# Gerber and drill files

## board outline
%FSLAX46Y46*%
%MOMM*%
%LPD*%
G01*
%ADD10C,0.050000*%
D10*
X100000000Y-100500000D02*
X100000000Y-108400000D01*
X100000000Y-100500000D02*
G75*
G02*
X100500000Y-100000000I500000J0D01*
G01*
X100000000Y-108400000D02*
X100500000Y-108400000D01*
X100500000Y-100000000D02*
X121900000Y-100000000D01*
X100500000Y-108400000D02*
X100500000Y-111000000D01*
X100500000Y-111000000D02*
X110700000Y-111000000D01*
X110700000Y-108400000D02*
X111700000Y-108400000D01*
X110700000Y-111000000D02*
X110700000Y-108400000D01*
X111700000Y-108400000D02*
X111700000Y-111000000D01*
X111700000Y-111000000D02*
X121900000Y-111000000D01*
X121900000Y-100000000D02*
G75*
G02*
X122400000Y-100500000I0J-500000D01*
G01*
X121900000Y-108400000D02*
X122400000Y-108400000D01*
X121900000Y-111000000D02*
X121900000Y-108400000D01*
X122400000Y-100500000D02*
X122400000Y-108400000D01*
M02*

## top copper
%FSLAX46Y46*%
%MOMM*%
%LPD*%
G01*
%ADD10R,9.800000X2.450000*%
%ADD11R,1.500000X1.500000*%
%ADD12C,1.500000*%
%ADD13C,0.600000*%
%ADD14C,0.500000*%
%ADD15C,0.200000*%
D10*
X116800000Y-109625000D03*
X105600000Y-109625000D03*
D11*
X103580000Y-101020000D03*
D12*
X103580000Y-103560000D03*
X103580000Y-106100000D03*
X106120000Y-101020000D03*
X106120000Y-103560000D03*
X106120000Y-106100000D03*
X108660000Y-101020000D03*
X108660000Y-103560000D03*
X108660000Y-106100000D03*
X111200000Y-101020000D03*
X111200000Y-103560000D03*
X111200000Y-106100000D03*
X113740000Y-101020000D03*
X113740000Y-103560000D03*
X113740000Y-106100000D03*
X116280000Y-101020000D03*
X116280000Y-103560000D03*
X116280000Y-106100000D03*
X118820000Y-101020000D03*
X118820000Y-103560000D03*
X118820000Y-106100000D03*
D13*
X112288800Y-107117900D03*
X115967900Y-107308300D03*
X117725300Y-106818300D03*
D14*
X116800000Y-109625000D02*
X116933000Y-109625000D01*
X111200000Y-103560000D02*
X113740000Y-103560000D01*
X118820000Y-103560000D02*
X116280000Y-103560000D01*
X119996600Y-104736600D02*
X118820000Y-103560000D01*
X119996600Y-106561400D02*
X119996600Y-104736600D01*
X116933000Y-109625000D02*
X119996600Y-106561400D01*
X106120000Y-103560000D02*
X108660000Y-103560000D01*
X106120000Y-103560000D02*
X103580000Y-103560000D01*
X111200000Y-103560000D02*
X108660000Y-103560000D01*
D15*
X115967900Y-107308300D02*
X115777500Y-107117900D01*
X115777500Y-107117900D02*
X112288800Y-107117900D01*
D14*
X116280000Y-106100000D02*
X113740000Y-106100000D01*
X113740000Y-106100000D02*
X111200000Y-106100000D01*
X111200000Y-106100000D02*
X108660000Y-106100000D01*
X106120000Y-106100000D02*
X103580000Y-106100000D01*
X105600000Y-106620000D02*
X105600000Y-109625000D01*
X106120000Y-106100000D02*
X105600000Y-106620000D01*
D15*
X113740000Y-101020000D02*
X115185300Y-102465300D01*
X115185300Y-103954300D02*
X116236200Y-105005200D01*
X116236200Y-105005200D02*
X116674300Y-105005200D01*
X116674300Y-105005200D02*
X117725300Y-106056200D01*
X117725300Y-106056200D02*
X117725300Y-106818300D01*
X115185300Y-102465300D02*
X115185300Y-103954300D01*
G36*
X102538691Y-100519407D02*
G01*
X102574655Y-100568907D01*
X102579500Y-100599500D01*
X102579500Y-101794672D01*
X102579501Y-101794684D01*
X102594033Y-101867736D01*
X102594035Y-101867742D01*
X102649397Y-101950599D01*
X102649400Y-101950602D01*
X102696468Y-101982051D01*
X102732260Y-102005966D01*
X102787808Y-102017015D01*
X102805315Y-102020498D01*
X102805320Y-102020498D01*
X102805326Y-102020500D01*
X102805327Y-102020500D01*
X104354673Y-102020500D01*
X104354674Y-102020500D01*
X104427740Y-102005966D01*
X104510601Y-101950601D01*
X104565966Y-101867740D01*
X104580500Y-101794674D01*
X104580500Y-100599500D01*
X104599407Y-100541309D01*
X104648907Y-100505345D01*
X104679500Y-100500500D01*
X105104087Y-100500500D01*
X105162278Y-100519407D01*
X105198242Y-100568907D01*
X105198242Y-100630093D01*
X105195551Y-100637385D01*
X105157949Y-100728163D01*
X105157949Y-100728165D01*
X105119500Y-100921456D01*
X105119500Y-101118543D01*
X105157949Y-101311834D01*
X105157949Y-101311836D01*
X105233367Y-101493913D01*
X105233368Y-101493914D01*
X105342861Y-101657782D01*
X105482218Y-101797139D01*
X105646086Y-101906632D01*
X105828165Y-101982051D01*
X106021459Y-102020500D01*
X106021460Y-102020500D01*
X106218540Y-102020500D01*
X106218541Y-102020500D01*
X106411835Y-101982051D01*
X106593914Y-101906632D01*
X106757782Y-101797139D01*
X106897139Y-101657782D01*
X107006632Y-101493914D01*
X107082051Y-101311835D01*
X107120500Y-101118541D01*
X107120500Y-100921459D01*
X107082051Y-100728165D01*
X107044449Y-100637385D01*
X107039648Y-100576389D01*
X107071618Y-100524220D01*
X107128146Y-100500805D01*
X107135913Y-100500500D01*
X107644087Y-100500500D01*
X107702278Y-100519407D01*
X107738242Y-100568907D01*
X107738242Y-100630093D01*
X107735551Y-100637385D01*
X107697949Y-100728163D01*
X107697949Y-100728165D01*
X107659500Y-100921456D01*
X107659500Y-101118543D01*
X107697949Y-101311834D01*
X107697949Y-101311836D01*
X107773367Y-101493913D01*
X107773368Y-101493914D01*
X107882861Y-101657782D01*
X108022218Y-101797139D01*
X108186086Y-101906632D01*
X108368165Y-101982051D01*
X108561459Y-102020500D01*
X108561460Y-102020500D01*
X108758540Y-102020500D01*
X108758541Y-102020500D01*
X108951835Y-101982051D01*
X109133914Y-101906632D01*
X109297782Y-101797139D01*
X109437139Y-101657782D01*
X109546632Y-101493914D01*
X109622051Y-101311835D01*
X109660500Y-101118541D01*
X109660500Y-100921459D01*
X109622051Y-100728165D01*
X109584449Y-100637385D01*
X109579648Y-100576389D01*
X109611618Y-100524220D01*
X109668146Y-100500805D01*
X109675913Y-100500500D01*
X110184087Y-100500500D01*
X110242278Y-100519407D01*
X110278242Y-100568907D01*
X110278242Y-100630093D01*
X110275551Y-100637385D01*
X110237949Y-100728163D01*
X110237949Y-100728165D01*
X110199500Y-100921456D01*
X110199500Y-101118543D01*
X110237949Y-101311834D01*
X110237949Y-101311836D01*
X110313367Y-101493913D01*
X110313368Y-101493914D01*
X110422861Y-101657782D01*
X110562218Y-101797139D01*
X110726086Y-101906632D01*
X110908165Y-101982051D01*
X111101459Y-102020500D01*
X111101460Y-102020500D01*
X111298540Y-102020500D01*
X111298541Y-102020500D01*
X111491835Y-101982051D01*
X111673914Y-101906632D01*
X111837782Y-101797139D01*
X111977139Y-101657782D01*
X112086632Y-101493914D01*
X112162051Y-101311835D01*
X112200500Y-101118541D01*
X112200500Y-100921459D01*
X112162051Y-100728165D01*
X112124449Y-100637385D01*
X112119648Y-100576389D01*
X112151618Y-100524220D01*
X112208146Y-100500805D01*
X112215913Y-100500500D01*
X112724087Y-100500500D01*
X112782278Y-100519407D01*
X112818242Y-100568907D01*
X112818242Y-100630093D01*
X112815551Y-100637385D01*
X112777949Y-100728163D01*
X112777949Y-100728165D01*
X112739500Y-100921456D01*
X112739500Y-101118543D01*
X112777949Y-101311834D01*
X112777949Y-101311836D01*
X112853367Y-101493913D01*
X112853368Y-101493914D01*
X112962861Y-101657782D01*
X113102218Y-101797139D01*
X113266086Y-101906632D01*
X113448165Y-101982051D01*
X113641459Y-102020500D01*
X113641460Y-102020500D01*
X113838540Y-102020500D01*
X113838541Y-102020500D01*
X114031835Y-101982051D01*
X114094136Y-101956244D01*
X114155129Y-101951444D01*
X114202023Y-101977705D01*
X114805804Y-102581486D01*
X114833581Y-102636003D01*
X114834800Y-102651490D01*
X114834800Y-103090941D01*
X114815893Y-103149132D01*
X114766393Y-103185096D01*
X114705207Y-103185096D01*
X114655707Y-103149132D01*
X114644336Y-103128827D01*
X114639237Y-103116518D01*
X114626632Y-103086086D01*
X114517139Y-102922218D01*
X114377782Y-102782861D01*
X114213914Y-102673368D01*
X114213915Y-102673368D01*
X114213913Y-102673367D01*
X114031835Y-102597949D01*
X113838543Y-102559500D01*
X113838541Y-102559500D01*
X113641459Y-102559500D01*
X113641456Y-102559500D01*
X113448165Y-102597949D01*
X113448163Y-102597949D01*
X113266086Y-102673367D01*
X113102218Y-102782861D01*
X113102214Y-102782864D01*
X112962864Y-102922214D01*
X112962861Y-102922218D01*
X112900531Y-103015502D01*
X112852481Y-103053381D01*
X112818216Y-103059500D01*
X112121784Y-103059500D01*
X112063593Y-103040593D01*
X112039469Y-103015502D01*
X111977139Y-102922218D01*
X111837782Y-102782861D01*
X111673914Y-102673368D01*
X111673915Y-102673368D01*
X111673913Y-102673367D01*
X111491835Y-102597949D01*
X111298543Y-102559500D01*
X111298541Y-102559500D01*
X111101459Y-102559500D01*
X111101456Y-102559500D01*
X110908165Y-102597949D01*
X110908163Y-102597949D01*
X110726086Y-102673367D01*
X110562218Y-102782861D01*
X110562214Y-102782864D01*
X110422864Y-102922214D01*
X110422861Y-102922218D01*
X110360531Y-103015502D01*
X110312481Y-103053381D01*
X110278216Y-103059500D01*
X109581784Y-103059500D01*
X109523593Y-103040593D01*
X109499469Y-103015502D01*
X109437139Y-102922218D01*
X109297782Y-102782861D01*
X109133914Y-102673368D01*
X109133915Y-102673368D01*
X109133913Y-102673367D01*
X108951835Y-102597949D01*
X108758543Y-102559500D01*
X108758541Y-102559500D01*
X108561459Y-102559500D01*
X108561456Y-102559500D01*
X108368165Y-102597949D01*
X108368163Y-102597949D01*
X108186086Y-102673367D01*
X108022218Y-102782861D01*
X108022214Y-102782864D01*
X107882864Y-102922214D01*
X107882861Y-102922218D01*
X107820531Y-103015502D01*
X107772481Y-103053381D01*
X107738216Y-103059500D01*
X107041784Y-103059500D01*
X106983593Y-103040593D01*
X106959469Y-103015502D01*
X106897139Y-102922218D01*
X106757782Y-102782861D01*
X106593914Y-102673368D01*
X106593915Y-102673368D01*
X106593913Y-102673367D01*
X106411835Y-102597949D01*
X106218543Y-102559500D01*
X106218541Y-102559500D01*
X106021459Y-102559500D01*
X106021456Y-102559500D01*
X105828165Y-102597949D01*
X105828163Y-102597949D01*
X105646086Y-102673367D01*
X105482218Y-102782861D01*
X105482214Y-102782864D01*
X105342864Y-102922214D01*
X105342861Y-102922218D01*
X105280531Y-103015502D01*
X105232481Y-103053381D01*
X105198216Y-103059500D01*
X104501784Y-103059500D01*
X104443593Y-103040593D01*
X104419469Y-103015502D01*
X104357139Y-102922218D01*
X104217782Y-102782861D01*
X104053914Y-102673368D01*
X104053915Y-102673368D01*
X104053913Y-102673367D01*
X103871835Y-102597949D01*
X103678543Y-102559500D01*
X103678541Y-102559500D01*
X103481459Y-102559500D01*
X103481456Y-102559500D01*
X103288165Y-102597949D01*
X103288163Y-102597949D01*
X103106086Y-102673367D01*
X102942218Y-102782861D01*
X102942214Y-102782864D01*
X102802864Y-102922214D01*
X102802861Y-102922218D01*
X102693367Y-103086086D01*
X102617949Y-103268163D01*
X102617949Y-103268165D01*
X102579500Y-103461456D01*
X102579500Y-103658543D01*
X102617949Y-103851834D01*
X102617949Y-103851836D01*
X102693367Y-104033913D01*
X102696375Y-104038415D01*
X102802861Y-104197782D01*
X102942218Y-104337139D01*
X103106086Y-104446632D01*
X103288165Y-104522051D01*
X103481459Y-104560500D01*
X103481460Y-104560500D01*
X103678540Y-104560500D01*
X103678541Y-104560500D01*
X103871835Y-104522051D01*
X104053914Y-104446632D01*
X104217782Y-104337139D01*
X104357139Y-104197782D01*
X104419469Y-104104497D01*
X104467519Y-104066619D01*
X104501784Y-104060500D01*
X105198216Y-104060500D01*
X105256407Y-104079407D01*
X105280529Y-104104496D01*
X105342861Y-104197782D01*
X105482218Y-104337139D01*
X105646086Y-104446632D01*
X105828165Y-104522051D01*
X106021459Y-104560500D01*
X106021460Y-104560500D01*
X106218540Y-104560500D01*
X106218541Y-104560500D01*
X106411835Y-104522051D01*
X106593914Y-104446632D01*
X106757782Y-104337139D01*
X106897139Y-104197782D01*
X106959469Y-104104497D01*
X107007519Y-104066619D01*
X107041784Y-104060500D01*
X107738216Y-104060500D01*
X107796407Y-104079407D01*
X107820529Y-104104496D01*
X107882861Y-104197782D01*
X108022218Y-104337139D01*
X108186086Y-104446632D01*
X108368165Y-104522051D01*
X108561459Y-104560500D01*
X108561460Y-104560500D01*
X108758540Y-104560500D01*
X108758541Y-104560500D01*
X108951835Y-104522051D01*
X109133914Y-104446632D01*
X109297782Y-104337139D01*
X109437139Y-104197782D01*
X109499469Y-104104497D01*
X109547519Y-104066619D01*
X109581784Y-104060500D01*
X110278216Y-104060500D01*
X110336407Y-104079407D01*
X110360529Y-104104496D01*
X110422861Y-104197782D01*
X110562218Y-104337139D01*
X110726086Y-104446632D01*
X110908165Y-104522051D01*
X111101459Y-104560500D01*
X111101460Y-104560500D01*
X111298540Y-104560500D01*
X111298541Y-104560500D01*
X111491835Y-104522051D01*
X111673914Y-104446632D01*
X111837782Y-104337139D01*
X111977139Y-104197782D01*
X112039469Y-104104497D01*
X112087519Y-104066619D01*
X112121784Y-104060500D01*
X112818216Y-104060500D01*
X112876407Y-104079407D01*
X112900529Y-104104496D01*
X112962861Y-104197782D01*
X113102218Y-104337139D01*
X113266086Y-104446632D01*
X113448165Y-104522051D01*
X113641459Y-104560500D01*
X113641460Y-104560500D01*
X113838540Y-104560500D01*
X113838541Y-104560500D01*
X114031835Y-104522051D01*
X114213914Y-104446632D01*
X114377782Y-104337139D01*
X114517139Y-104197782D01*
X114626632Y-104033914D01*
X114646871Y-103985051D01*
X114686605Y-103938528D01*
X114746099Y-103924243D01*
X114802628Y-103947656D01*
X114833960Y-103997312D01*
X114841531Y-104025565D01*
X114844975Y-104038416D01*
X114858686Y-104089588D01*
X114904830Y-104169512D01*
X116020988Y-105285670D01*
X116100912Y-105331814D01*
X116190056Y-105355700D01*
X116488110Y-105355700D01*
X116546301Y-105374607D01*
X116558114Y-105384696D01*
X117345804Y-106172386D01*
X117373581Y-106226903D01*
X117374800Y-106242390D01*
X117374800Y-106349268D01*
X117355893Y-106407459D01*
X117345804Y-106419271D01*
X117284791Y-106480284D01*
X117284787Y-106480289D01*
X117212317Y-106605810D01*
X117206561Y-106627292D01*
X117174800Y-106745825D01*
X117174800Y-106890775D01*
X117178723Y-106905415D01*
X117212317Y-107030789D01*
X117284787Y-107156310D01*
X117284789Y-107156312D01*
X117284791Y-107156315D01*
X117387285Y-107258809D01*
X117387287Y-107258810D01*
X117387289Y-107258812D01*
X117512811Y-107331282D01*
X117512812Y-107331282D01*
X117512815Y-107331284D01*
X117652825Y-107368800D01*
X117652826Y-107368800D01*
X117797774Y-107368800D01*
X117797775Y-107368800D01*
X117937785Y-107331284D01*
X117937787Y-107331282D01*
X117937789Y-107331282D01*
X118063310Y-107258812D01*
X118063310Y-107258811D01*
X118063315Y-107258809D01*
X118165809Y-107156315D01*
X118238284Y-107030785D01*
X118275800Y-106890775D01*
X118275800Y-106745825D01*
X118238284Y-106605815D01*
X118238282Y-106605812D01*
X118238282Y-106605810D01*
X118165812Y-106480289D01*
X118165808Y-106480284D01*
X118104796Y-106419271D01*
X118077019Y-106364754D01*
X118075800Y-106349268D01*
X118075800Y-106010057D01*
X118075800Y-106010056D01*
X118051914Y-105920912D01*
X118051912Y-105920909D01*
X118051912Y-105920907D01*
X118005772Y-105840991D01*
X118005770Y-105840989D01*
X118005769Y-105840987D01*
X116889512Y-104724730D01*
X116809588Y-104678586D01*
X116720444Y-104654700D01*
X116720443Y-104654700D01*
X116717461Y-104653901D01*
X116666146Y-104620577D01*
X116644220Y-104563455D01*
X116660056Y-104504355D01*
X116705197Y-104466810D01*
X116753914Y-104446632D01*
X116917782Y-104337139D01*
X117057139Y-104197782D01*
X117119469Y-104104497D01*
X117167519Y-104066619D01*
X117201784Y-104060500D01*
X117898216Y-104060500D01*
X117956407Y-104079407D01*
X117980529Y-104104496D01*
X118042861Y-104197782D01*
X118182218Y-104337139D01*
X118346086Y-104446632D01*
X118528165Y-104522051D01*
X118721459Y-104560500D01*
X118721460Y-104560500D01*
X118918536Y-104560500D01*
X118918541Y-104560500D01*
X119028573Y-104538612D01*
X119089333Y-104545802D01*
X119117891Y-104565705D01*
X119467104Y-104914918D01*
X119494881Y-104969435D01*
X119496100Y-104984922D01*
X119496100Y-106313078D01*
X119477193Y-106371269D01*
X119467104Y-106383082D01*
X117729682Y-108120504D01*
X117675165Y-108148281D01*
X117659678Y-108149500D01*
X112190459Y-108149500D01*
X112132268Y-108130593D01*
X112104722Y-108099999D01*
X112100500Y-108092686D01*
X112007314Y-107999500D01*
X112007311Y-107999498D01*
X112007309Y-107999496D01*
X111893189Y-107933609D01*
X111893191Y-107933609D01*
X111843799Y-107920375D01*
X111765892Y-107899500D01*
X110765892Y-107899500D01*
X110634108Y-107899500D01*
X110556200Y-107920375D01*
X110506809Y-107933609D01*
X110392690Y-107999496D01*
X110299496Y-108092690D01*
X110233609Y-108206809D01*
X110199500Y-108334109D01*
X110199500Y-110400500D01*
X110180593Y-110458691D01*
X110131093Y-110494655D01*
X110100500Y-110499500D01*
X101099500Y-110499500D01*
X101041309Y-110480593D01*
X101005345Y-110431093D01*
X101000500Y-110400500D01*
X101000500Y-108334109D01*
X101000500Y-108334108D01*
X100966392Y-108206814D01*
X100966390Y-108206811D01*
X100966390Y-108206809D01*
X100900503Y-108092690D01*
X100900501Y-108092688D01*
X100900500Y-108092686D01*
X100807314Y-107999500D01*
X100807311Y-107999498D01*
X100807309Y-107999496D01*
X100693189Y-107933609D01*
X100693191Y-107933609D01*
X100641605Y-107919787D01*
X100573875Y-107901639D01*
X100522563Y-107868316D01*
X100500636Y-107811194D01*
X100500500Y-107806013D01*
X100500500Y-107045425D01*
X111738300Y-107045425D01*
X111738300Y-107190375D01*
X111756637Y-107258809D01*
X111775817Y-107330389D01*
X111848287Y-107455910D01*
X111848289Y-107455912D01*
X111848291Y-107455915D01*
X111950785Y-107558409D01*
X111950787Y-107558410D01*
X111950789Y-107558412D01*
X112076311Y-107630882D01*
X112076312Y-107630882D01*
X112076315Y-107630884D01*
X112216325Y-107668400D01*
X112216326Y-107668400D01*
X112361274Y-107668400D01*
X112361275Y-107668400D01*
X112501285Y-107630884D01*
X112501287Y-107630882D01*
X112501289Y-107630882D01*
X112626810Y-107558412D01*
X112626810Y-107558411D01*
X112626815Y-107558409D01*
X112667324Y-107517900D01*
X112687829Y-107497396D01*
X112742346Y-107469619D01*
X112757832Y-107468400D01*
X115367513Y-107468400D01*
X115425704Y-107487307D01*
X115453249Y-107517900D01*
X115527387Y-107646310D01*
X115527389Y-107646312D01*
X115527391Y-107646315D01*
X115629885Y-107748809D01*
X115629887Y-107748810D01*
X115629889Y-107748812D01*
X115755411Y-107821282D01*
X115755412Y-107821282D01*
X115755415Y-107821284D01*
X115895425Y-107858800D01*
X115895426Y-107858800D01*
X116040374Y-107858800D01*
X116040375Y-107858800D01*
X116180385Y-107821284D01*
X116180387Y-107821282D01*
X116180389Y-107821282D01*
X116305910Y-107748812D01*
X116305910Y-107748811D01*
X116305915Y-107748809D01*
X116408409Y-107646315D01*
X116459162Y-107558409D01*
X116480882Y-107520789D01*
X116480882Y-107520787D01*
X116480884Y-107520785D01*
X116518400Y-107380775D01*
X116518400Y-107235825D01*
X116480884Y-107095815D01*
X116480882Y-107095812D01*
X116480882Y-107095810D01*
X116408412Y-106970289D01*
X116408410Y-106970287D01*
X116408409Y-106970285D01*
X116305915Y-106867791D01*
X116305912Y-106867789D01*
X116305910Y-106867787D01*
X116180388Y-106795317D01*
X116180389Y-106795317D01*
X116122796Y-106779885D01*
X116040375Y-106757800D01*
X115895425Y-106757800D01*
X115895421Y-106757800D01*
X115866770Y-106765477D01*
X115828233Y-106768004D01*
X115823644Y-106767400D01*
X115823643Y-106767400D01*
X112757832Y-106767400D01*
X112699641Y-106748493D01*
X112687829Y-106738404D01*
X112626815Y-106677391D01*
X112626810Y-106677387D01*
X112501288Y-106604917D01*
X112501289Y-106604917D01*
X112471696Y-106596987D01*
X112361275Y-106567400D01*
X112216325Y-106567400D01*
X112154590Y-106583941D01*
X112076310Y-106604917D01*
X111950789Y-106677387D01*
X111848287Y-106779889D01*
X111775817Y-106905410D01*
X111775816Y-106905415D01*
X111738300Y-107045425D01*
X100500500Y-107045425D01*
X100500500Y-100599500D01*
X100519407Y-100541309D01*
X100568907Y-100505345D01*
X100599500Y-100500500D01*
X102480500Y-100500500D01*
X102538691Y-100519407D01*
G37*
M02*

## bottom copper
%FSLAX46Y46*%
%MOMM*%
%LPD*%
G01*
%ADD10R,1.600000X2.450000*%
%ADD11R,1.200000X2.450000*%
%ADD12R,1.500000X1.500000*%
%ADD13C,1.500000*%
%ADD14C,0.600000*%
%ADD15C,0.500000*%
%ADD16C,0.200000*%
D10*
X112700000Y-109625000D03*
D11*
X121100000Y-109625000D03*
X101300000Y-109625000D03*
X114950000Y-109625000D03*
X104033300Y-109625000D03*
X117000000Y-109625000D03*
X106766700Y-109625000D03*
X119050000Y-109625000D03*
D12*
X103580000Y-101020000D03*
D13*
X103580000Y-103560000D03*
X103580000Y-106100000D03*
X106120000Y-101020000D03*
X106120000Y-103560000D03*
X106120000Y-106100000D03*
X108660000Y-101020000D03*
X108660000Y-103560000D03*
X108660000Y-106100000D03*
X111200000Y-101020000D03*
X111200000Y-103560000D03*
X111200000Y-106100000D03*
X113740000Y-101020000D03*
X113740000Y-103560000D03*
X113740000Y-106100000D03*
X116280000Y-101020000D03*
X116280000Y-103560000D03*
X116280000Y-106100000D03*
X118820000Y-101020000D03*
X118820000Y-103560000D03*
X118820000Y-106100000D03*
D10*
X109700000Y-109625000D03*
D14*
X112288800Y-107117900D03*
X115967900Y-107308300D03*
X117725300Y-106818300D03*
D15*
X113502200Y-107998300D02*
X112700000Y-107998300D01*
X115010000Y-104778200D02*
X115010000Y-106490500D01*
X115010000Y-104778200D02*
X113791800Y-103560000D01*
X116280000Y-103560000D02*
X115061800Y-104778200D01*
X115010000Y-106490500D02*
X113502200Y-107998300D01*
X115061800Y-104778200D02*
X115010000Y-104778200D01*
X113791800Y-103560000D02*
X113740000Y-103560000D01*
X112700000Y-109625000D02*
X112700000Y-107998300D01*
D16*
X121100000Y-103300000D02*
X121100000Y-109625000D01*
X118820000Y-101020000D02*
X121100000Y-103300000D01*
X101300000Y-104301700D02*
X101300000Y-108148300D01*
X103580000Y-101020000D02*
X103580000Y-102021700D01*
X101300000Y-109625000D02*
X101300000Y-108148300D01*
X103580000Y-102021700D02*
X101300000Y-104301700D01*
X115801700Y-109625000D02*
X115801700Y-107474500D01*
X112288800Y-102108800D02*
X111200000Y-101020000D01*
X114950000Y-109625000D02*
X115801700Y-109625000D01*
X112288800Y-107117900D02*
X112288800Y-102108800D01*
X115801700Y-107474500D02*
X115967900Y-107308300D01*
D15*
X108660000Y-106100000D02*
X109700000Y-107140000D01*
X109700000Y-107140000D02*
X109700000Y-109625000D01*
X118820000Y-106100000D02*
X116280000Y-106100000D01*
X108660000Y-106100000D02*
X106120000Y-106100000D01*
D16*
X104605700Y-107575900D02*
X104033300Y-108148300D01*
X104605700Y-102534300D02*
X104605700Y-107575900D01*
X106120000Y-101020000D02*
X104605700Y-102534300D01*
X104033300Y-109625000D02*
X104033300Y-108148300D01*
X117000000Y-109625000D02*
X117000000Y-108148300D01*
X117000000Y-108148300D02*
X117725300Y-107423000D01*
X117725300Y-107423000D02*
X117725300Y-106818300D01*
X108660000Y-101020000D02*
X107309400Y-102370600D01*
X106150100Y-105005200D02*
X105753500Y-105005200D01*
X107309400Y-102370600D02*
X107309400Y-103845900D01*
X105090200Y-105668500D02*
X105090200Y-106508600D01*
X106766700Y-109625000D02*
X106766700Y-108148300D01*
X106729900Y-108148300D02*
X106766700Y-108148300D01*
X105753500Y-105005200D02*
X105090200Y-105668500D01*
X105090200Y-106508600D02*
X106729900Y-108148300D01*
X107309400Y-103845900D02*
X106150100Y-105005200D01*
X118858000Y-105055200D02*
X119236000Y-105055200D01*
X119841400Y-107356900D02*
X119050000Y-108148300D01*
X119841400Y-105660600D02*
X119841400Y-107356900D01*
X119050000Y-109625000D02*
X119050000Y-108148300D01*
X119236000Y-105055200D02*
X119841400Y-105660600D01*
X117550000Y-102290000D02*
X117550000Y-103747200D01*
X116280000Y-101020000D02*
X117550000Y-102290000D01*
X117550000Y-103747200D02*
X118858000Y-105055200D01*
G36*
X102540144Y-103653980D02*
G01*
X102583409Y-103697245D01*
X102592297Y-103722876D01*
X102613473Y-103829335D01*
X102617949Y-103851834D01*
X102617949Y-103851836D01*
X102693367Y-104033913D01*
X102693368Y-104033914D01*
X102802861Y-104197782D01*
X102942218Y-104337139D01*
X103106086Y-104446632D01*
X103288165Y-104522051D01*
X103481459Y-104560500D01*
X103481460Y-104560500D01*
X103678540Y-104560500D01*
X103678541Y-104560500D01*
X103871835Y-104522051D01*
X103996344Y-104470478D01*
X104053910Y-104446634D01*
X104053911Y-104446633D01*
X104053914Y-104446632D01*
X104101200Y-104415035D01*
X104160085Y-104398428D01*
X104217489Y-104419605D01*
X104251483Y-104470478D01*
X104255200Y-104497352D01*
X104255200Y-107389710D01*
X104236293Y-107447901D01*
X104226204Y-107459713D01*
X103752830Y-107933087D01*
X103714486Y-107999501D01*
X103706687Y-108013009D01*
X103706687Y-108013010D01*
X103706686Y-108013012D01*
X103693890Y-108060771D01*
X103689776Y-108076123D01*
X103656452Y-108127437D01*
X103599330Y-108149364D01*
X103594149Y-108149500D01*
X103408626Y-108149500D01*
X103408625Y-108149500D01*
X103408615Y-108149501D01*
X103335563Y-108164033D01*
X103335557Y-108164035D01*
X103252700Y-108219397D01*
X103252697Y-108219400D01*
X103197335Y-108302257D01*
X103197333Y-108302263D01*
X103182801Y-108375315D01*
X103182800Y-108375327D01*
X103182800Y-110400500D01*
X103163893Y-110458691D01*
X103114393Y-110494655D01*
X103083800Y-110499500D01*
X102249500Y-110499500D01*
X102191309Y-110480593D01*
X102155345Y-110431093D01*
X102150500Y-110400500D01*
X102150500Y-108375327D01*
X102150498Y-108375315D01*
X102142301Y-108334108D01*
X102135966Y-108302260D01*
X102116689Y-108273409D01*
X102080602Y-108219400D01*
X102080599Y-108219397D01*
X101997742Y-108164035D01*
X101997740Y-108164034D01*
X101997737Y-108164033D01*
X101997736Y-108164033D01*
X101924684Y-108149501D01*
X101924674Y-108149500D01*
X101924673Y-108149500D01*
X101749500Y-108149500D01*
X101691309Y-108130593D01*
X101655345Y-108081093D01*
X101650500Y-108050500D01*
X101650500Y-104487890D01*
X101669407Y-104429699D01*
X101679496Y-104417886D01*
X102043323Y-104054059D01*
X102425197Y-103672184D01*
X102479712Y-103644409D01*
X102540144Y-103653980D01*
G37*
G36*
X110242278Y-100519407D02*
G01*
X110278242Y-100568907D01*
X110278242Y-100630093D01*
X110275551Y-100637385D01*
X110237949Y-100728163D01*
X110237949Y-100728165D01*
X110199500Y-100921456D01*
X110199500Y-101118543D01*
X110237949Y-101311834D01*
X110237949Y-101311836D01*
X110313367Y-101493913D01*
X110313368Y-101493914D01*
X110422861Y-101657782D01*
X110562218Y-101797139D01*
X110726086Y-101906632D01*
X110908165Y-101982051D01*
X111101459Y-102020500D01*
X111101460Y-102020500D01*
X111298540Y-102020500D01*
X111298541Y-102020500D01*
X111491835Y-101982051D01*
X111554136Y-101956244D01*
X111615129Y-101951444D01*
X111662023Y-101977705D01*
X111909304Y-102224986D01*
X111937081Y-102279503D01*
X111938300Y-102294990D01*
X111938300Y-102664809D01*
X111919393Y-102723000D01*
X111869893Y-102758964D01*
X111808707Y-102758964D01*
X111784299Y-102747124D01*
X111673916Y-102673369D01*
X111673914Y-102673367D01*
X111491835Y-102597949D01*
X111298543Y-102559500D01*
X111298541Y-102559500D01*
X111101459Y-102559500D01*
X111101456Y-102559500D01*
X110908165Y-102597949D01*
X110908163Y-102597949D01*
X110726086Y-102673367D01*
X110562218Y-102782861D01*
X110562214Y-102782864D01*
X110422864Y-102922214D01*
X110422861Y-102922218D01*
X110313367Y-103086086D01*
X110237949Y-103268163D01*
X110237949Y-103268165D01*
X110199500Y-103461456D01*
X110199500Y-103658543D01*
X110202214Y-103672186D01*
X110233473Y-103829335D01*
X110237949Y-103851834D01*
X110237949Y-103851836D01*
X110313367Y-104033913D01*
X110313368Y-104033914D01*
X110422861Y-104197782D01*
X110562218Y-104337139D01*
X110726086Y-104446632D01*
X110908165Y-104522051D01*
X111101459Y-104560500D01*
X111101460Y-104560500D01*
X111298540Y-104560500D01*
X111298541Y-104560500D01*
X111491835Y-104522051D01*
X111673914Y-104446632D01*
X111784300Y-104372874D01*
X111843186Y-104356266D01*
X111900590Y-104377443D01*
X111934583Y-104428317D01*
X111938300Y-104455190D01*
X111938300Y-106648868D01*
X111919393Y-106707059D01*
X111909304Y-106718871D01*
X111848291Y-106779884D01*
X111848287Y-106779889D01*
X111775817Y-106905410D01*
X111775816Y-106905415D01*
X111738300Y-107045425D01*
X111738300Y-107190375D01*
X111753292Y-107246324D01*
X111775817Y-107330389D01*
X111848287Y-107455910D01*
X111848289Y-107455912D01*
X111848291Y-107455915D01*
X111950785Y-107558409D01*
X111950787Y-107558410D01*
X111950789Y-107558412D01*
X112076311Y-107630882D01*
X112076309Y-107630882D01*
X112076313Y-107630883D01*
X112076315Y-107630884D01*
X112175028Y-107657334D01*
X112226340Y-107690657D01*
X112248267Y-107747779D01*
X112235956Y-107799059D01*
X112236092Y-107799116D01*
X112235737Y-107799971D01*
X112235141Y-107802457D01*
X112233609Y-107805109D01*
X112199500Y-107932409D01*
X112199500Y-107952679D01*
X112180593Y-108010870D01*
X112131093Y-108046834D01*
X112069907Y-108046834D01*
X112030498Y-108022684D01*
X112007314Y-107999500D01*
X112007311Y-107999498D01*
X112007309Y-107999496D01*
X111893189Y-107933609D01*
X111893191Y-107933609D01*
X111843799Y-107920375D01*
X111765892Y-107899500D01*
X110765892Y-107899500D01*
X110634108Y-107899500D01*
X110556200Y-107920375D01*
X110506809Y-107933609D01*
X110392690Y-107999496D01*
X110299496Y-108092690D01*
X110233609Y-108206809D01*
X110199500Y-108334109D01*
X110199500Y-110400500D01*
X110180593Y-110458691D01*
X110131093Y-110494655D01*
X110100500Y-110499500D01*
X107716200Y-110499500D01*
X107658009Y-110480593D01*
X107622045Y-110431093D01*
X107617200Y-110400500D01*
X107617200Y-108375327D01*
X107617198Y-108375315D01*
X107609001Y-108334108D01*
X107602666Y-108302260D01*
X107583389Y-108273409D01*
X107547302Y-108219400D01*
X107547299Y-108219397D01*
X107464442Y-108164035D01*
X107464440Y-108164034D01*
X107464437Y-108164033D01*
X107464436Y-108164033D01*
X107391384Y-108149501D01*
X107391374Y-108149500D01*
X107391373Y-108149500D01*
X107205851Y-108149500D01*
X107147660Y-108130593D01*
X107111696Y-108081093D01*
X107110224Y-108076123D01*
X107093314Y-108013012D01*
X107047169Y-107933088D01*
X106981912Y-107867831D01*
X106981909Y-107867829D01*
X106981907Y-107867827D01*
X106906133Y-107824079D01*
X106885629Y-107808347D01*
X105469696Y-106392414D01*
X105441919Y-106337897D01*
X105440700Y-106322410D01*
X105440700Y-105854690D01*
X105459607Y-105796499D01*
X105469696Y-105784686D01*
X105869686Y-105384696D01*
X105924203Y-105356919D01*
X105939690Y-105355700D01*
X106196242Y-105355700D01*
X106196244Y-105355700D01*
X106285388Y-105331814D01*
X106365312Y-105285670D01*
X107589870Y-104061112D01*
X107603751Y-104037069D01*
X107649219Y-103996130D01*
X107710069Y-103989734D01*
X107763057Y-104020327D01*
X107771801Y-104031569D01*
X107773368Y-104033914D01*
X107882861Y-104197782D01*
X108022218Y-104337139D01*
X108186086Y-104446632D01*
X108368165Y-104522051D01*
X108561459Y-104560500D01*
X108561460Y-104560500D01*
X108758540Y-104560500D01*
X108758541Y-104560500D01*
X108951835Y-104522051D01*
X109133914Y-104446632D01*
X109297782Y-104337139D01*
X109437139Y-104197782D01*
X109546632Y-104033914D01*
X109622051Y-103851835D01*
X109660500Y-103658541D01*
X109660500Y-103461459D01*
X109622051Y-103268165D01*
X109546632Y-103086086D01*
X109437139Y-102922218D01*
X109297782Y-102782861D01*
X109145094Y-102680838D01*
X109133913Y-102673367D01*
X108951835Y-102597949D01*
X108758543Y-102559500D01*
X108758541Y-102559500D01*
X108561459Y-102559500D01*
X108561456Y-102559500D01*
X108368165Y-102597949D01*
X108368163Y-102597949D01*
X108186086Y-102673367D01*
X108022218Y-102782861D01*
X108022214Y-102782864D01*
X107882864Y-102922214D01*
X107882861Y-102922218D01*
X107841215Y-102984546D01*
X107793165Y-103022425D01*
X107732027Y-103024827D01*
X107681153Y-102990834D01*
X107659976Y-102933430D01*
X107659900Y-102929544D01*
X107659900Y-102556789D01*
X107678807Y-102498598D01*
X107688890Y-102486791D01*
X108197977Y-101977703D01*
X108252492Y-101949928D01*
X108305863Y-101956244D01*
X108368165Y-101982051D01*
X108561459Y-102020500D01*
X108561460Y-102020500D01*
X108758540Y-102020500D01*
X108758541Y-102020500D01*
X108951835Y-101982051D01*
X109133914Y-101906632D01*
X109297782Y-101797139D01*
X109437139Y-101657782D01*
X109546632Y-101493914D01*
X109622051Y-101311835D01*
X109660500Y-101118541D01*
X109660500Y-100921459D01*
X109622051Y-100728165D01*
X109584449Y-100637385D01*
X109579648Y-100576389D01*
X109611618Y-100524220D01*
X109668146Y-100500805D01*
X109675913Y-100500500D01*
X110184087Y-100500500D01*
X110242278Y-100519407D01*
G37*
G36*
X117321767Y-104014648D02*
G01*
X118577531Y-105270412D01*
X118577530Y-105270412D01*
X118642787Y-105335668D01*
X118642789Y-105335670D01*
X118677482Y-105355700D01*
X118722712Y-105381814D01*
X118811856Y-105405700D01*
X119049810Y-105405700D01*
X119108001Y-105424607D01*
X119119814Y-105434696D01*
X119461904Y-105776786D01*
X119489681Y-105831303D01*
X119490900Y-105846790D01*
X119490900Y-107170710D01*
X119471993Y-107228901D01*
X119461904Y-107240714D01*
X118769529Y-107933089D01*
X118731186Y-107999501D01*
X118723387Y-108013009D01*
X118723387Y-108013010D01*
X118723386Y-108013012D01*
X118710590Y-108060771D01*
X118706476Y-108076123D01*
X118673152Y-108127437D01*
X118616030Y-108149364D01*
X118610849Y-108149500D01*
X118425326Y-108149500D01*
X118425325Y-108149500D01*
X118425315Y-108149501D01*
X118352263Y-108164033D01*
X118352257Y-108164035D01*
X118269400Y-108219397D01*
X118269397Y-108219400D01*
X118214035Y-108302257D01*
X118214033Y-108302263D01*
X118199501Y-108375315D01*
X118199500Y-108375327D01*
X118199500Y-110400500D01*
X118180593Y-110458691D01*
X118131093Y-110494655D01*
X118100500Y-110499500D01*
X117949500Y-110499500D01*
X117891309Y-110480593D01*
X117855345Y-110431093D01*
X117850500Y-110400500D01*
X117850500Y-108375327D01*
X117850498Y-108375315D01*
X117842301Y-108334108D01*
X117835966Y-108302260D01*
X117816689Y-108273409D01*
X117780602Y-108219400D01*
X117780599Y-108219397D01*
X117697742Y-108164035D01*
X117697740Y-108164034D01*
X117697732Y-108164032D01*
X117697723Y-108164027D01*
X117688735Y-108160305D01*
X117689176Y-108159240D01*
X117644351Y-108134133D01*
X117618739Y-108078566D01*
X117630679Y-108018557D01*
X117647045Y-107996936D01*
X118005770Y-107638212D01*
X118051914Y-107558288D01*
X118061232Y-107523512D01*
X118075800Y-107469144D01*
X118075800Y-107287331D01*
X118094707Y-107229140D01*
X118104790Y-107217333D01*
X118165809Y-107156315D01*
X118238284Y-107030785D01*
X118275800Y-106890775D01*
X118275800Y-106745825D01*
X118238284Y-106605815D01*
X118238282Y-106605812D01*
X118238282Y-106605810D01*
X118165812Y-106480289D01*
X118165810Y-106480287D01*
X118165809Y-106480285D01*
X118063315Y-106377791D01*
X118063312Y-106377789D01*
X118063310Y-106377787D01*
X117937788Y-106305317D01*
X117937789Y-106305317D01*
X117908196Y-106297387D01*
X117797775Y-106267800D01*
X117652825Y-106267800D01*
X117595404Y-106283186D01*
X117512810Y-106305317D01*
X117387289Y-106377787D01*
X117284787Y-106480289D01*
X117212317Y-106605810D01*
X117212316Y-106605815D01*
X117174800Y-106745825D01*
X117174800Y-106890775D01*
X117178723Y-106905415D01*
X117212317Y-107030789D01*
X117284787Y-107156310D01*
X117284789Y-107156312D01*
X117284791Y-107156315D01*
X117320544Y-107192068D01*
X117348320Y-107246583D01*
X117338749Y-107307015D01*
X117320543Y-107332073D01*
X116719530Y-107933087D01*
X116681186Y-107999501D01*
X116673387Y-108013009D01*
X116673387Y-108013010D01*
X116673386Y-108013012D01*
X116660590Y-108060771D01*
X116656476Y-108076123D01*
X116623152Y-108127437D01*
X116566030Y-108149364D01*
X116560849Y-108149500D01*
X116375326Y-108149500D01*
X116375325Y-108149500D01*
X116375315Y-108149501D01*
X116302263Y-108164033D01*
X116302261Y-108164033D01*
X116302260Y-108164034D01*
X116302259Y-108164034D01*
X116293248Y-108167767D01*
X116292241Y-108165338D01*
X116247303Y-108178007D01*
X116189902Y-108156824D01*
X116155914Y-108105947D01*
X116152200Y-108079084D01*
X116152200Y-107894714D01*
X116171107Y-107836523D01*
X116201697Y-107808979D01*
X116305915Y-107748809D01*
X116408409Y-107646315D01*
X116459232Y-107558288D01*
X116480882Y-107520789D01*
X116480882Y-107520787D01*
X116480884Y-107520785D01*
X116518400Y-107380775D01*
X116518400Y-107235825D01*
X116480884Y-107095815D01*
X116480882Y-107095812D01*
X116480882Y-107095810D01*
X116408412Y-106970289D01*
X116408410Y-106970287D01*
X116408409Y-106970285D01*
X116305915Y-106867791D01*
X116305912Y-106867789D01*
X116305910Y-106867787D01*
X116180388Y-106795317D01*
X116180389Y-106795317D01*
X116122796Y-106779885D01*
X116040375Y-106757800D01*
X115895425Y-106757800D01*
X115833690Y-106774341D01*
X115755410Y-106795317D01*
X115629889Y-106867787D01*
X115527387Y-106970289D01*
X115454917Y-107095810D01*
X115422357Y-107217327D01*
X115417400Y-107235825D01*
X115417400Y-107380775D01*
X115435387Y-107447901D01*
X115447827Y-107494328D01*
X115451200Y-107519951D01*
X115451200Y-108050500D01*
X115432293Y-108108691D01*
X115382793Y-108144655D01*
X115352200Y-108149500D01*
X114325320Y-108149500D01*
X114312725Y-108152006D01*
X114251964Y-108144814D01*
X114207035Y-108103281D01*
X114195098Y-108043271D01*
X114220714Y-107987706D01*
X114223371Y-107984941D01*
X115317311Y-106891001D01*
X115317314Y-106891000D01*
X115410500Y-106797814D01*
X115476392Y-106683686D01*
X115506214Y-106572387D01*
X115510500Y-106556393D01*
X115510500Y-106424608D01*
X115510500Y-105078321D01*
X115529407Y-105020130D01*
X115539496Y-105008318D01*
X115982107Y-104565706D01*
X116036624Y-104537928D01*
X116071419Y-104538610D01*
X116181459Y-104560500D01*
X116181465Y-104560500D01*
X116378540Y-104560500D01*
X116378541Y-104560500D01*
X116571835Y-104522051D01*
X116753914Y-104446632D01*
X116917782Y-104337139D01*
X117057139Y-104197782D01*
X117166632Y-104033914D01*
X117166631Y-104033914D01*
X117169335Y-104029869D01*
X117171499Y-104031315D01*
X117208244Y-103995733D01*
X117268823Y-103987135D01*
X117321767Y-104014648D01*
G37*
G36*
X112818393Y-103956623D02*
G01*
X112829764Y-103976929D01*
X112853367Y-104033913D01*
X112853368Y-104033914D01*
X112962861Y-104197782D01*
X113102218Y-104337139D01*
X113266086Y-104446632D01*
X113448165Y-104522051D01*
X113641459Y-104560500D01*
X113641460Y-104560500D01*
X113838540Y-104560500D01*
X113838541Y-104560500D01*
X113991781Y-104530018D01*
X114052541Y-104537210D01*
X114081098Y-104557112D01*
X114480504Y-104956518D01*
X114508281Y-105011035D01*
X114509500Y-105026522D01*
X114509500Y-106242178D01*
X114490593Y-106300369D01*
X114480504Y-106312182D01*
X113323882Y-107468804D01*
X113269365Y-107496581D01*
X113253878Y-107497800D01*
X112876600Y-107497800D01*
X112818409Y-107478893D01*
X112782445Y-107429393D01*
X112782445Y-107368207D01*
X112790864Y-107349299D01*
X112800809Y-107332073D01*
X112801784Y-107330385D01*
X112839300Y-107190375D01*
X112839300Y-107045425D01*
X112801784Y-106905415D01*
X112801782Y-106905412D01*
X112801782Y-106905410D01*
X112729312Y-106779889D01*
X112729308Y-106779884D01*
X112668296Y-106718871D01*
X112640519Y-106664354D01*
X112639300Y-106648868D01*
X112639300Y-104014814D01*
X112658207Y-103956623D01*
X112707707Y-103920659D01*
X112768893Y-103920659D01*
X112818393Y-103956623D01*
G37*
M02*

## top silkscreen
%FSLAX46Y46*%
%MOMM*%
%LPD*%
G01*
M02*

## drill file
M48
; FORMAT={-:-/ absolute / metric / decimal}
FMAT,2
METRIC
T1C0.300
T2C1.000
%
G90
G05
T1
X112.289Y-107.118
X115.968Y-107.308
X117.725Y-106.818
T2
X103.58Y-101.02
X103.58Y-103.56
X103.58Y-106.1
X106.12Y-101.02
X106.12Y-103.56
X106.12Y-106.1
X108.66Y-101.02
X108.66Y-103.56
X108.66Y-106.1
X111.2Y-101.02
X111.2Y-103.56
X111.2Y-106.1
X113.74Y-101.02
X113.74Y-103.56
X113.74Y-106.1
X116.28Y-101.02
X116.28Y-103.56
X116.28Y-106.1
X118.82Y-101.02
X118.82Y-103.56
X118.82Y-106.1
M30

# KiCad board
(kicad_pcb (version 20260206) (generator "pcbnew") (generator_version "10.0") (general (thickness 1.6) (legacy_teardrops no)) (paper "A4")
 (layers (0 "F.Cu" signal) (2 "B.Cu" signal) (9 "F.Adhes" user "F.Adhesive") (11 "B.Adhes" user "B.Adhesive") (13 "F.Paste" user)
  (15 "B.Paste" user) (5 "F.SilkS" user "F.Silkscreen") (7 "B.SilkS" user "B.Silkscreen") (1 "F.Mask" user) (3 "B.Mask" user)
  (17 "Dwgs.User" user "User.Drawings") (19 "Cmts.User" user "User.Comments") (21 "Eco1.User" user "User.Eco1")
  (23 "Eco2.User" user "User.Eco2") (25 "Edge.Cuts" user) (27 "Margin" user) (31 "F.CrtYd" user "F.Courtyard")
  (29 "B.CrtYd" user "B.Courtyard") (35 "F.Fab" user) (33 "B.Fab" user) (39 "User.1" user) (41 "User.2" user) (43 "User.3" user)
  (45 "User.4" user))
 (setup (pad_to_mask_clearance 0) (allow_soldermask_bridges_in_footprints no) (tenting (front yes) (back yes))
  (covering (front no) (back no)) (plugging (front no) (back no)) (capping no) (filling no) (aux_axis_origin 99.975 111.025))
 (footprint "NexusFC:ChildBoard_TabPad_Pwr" (layer "F.Cu") (at 112.7 108.4)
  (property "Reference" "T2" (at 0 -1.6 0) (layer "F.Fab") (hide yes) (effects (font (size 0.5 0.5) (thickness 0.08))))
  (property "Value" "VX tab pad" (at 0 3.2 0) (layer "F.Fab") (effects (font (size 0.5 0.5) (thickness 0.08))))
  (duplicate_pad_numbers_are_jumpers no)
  (pad "1" smd rect (at 0 1.225) (size 1.6 2.45) (layers "B.Cu" "B.Mask") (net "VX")))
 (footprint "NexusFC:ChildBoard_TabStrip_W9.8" (layer "F.Cu") (at 116.8 108.4)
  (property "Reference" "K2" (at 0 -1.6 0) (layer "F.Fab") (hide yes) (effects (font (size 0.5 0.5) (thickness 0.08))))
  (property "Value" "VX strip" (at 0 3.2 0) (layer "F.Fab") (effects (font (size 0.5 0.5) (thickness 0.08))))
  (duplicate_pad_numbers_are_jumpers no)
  (pad "1" smd rect (at 0 1.225) (size 9.8 2.45) (layers "F.Cu" "F.Mask") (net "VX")))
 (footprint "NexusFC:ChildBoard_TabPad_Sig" (layer "F.Cu") (at 121.1 108.4)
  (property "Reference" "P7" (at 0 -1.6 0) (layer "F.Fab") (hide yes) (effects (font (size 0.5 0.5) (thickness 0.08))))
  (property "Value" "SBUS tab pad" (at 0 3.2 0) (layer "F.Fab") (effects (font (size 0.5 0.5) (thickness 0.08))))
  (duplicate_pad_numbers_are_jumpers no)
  (pad "1" smd rect (at 0 1.225) (size 1.2 2.45) (layers "B.Cu" "B.Mask") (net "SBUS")))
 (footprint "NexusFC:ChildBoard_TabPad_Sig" (layer "F.Cu") (at 101.3 108.4)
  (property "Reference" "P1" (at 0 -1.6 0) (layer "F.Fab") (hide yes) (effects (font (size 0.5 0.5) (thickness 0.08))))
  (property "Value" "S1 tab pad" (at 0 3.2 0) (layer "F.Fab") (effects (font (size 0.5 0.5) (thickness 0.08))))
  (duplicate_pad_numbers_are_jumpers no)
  (pad "1" smd rect (at 0 1.225) (size 1.2 2.45) (layers "B.Cu" "B.Mask") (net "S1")))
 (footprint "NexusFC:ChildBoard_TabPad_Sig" (layer "F.Cu") (at 114.95 108.4)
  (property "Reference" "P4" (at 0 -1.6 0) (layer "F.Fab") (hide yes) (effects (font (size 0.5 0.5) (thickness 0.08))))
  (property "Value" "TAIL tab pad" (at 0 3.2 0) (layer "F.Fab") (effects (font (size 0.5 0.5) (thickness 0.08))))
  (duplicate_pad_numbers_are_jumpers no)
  (pad "1" smd rect (at 0 1.225) (size 1.2 2.45) (layers "B.Cu" "B.Mask") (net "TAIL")))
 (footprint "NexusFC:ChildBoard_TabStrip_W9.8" (layer "F.Cu") (at 105.6 108.4)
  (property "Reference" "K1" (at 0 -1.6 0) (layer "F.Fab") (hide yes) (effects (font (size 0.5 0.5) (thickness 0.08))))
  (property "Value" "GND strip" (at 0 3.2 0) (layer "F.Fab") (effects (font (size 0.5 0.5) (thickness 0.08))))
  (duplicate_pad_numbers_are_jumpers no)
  (pad "1" smd rect (at 0 1.225) (size 9.8 2.45) (layers "F.Cu" "F.Mask") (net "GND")))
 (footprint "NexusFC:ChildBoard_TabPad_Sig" (layer "F.Cu") (at 104.0333 108.4)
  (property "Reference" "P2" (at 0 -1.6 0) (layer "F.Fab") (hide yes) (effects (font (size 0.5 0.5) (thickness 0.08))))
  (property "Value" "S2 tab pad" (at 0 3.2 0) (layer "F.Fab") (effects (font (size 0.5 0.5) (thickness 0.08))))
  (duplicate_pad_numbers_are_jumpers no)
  (pad "1" smd rect (at 0 1.225) (size 1.2 2.45) (layers "B.Cu" "B.Mask") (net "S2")))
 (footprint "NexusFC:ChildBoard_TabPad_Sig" (layer "F.Cu") (at 117 108.4)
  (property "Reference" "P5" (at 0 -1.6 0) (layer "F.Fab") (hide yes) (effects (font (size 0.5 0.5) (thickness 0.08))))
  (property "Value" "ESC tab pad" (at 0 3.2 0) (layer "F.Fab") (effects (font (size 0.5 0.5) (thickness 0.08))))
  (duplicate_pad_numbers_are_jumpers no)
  (pad "1" smd rect (at 0 1.225) (size 1.2 2.45) (layers "B.Cu" "B.Mask") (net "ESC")))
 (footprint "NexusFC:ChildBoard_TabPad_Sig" (layer "F.Cu") (at 106.7667 108.4)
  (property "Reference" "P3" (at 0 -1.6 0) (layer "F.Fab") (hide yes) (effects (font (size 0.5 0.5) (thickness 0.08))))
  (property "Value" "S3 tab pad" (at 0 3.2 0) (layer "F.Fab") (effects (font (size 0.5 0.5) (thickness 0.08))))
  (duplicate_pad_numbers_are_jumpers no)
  (pad "1" smd rect (at 0 1.225) (size 1.2 2.45) (layers "B.Cu" "B.Mask") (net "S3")))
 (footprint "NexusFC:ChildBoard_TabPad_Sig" (layer "F.Cu") (at 119.05 108.4)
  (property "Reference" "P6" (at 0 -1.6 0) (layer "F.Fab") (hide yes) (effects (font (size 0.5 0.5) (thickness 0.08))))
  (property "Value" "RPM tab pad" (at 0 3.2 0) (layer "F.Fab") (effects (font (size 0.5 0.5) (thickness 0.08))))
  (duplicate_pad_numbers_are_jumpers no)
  (pad "1" smd rect (at 0 1.225) (size 1.2 2.45) (layers "B.Cu" "B.Mask") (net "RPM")))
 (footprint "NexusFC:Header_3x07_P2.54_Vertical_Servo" (layer "F.Cu") (at 111.2 103.56)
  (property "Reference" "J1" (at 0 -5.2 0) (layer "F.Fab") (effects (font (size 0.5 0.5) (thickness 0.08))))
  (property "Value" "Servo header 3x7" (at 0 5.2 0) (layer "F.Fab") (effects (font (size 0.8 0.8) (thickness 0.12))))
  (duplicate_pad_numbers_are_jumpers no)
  (pad "1" thru_hole rect (at -7.62 -2.54) (size 1.5 1.5) (drill 1) (layers "*.Cu" "*.Mask") (remove_unused_layers no) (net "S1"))
  (pad "2" thru_hole circle (at -7.62 0) (size 1.5 1.5) (drill 1) (layers "*.Cu" "*.Mask") (remove_unused_layers no) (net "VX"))
  (pad "3" thru_hole circle (at -7.62 2.54) (size 1.5 1.5) (drill 1) (layers "*.Cu" "*.Mask") (remove_unused_layers no) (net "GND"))
  (pad "4" thru_hole circle (at -5.08 -2.54) (size 1.5 1.5) (drill 1) (layers "*.Cu" "*.Mask") (remove_unused_layers no) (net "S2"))
  (pad "5" thru_hole circle (at -5.08 0) (size 1.5 1.5) (drill 1) (layers "*.Cu" "*.Mask") (remove_unused_layers no) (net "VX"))
  (pad "6" thru_hole circle (at -5.08 2.54) (size 1.5 1.5) (drill 1) (layers "*.Cu" "*.Mask") (remove_unused_layers no) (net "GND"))
  (pad "7" thru_hole circle (at -2.54 -2.54) (size 1.5 1.5) (drill 1) (layers "*.Cu" "*.Mask") (remove_unused_layers no) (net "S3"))
  (pad "8" thru_hole circle (at -2.54 0) (size 1.5 1.5) (drill 1) (layers "*.Cu" "*.Mask") (remove_unused_layers no) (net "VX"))
  (pad "9" thru_hole circle (at -2.54 2.54) (size 1.5 1.5) (drill 1) (layers "*.Cu" "*.Mask") (remove_unused_layers no) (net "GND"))
  (pad "10" thru_hole circle (at 0 -2.54) (size 1.5 1.5) (drill 1) (layers "*.Cu" "*.Mask") (remove_unused_layers no) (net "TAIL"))
  (pad "11" thru_hole circle (at 0 0) (size 1.5 1.5) (drill 1) (layers "*.Cu" "*.Mask") (remove_unused_layers no) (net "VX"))
  (pad "12" thru_hole circle (at 0 2.54) (size 1.5 1.5) (drill 1) (layers "*.Cu" "*.Mask") (remove_unused_layers no) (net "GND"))
  (pad "13" thru_hole circle (at 2.54 -2.54) (size 1.5 1.5) (drill 1) (layers "*.Cu" "*.Mask") (remove_unused_layers no) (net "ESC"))
  (pad "14" thru_hole circle (at 2.54 0) (size 1.5 1.5) (drill 1) (layers "*.Cu" "*.Mask") (remove_unused_layers no) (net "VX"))
  (pad "15" thru_hole circle (at 2.54 2.54) (size 1.5 1.5) (drill 1) (layers "*.Cu" "*.Mask") (remove_unused_layers no) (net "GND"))
  (pad "16" thru_hole circle (at 5.08 -2.54) (size 1.5 1.5) (drill 1) (layers "*.Cu" "*.Mask") (remove_unused_layers no) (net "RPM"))
  (pad "17" thru_hole circle (at 5.08 0) (size 1.5 1.5) (drill 1) (layers "*.Cu" "*.Mask") (remove_unused_layers no) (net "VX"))
  (pad "18" thru_hole circle (at 5.08 2.54) (size 1.5 1.5) (drill 1) (layers "*.Cu" "*.Mask") (remove_unused_layers no) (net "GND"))
  (pad "19" thru_hole circle (at 7.62 -2.54) (size 1.5 1.5) (drill 1) (layers "*.Cu" "*.Mask") (remove_unused_layers no) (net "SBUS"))
  (pad "20" thru_hole circle (at 7.62 0) (size 1.5 1.5) (drill 1) (layers "*.Cu" "*.Mask") (remove_unused_layers no) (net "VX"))
  (pad "21" thru_hole circle (at 7.62 2.54) (size 1.5 1.5) (drill 1) (layers "*.Cu" "*.Mask") (remove_unused_layers no) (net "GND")))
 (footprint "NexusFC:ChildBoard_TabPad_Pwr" (layer "F.Cu") (at 109.7 108.4)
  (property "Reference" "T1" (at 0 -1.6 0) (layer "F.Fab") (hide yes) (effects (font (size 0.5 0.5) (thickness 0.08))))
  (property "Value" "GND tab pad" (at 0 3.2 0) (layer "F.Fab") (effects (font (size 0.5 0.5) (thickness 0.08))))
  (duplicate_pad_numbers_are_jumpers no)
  (pad "1" smd rect (at 0 1.225) (size 1.6 2.45) (layers "B.Cu" "B.Mask") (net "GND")))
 (gr_line (start 100 100.5) (end 100 108.4) (stroke (width 0.05) (type default)) (layer "Edge.Cuts"))
 (gr_arc (start 100 100.5) (mid 100.146447 100.146447) (end 100.5 100) (stroke (width 0.05) (type default)) (layer "Edge.Cuts"))
 (gr_line (start 100 108.4) (end 100.5 108.4) (stroke (width 0.05) (type default)) (layer "Edge.Cuts"))
 (gr_line (start 100.5 100) (end 121.9 100) (stroke (width 0.05) (type default)) (layer "Edge.Cuts"))
 (gr_line (start 100.5 108.4) (end 100.5 111) (stroke (width 0.05) (type default)) (layer "Edge.Cuts"))
 (gr_line (start 100.5 111) (end 110.7 111) (stroke (width 0.05) (type default)) (layer "Edge.Cuts"))
 (gr_line (start 110.7 108.4) (end 111.7 108.4) (stroke (width 0.05) (type default)) (layer "Edge.Cuts"))
 (gr_line (start 110.7 111) (end 110.7 108.4) (stroke (width 0.05) (type default)) (layer "Edge.Cuts"))
 (gr_line (start 111.7 108.4) (end 111.7 111) (stroke (width 0.05) (type default)) (layer "Edge.Cuts"))
 (gr_line (start 111.7 111) (end 121.9 111) (stroke (width 0.05) (type default)) (layer "Edge.Cuts"))
 (gr_arc (start 121.9 100) (mid 122.253553 100.146447) (end 122.4 100.5) (stroke (width 0.05) (type default)) (layer "Edge.Cuts"))
 (gr_line (start 121.9 108.4) (end 122.4 108.4) (stroke (width 0.05) (type default)) (layer "Edge.Cuts"))
 (gr_line (start 121.9 111) (end 121.9 108.4) (stroke (width 0.05) (type default)) (layer "Edge.Cuts"))
 (gr_line (start 122.4 100.5) (end 122.4 108.4) (stroke (width 0.05) (type default)) (layer "Edge.Cuts"))
 (segment (start 116.8 109.625) (end 116.933 109.625) (width 0.5) (layer "F.Cu") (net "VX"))
 (segment (start 111.2 103.56) (end 113.74 103.56) (width 0.5) (layer "F.Cu") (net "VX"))
 (segment (start 118.82 103.56) (end 116.28 103.56) (width 0.5) (layer "F.Cu") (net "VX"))
 (segment (start 119.9966 104.7366) (end 118.82 103.56) (width 0.5) (layer "F.Cu") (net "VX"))
 (segment (start 119.9966 106.5614) (end 119.9966 104.7366) (width 0.5) (layer "F.Cu") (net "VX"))
 (segment (start 116.933 109.625) (end 119.9966 106.5614) (width 0.5) (layer "F.Cu") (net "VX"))
 (segment (start 106.12 103.56) (end 108.66 103.56) (width 0.5) (layer "F.Cu") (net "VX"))
 (segment (start 106.12 103.56) (end 103.58 103.56) (width 0.5) (layer "F.Cu") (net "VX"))
 (segment (start 111.2 103.56) (end 108.66 103.56) (width 0.5) (layer "F.Cu") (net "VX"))
 (segment (start 113.5022 107.9983) (end 112.7 107.9983) (width 0.5) (layer "B.Cu") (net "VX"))
 (segment (start 115.01 104.7782) (end 115.01 106.4905) (width 0.5) (layer "B.Cu") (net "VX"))
 (segment (start 115.01 104.7782) (end 113.7918 103.56) (width 0.5) (layer "B.Cu") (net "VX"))
 (segment (start 116.28 103.56) (end 115.0618 104.7782) (width 0.5) (layer "B.Cu") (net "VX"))
 (segment (start 115.01 106.4905) (end 113.5022 107.9983) (width 0.5) (layer "B.Cu") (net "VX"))
 (segment (start 115.0618 104.7782) (end 115.01 104.7782) (width 0.5) (layer "B.Cu") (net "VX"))
 (segment (start 113.7918 103.56) (end 113.74 103.56) (width 0.5) (layer "B.Cu") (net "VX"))
 (segment (start 112.7 109.625) (end 112.7 107.9983) (width 0.5) (layer "B.Cu") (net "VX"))
 (segment (start 121.1 103.3) (end 121.1 109.625) (width 0.2) (layer "B.Cu") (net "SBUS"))
 (segment (start 118.82 101.02) (end 121.1 103.3) (width 0.2) (layer "B.Cu") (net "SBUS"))
 (segment (start 101.3 104.3017) (end 101.3 108.1483) (width 0.2) (layer "B.Cu") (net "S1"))
 (segment (start 103.58 101.02) (end 103.58 102.0217) (width 0.2) (layer "B.Cu") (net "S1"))
 (segment (start 101.3 109.625) (end 101.3 108.1483) (width 0.2) (layer "B.Cu") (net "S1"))
 (segment (start 103.58 102.0217) (end 101.3 104.3017) (width 0.2) (layer "B.Cu") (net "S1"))
 (segment (start 115.9679 107.3083) (end 115.7775 107.1179) (width 0.2) (layer "F.Cu") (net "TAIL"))
 (segment (start 115.7775 107.1179) (end 112.2888 107.1179) (width 0.2) (layer "F.Cu") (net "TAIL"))
 (via (at 112.2888 107.1179) (size 0.6) (drill 0.3) (layers "F.Cu" "B.Cu") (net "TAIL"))
 (via (at 115.9679 107.3083) (size 0.6) (drill 0.3) (layers "F.Cu" "B.Cu") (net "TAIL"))
 (segment (start 115.8017 109.625) (end 115.8017 107.4745) (width 0.2) (layer "B.Cu") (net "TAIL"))
 (segment (start 112.2888 102.1088) (end 111.2 101.02) (width 0.2) (layer "B.Cu") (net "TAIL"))
 (segment (start 114.95 109.625) (end 115.8017 109.625) (width 0.2) (layer "B.Cu") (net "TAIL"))
 (segment (start 112.2888 107.1179) (end 112.2888 102.1088) (width 0.2) (layer "B.Cu") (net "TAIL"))
 (segment (start 115.8017 107.4745) (end 115.9679 107.3083) (width 0.2) (layer "B.Cu") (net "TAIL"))
 (segment (start 116.28 106.1) (end 113.74 106.1) (width 0.5) (layer "F.Cu") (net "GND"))
 (segment (start 113.74 106.1) (end 111.2 106.1) (width 0.5) (layer "F.Cu") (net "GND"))
 (segment (start 111.2 106.1) (end 108.66 106.1) (width 0.5) (layer "F.Cu") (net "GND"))
 (segment (start 106.12 106.1) (end 103.58 106.1) (width 0.5) (layer "F.Cu") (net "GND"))
 (segment (start 105.6 106.62) (end 105.6 109.625) (width 0.5) (layer "F.Cu") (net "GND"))
 (segment (start 106.12 106.1) (end 105.6 106.62) (width 0.5) (layer "F.Cu") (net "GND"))
 (segment (start 108.66 106.1) (end 109.7 107.14) (width 0.5) (layer "B.Cu") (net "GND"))
 (segment (start 109.7 107.14) (end 109.7 109.625) (width 0.5) (layer "B.Cu") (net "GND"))
 (segment (start 118.82 106.1) (end 116.28 106.1) (width 0.5) (layer "B.Cu") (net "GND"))
 (segment (start 108.66 106.1) (end 106.12 106.1) (width 0.5) (layer "B.Cu") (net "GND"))
 (segment (start 104.6057 107.5759) (end 104.0333 108.1483) (width 0.2) (layer "B.Cu") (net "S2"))
 (segment (start 104.6057 102.5343) (end 104.6057 107.5759) (width 0.2) (layer "B.Cu") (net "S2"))
 (segment (start 106.12 101.02) (end 104.6057 102.5343) (width 0.2) (layer "B.Cu") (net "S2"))
 (segment (start 104.0333 109.625) (end 104.0333 108.1483) (width 0.2) (layer "B.Cu") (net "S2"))
 (segment (start 113.74 101.02) (end 115.1853 102.4653) (width 0.2) (layer "F.Cu") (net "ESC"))
 (segment (start 115.1853 103.9543) (end 116.2362 105.0052) (width 0.2) (layer "F.Cu") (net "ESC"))
 (segment (start 116.2362 105.0052) (end 116.6743 105.0052) (width 0.2) (layer "F.Cu") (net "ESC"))
 (segment (start 116.6743 105.0052) (end 117.7253 106.0562) (width 0.2) (layer "F.Cu") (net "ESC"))
 (segment (start 117.7253 106.0562) (end 117.7253 106.8183) (width 0.2) (layer "F.Cu") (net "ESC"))
 (segment (start 115.1853 102.4653) (end 115.1853 103.9543) (width 0.2) (layer "F.Cu") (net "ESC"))
 (via (at 117.7253 106.8183) (size 0.6) (drill 0.3) (layers "F.Cu" "B.Cu") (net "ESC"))
 (segment (start 117 109.625) (end 117 108.1483) (width 0.2) (layer "B.Cu") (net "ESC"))
 (segment (start 117 108.1483) (end 117.7253 107.423) (width 0.2) (layer "B.Cu") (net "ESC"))
 (segment (start 117.7253 107.423) (end 117.7253 106.8183) (width 0.2) (layer "B.Cu") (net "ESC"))
 (segment (start 108.66 101.02) (end 107.3094 102.3706) (width 0.2) (layer "B.Cu") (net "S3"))
 (segment (start 106.1501 105.0052) (end 105.7535 105.0052) (width 0.2) (layer "B.Cu") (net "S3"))
 (segment (start 107.3094 102.3706) (end 107.3094 103.8459) (width 0.2) (layer "B.Cu") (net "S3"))
 (segment (start 105.0902 105.6685) (end 105.0902 106.5086) (width 0.2) (layer "B.Cu") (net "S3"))
 (segment (start 106.7667 109.625) (end 106.7667 108.1483) (width 0.2) (layer "B.Cu") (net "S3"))
 (segment (start 106.7299 108.1483) (end 106.7667 108.1483) (width 0.2) (layer "B.Cu") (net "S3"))
 (segment (start 105.7535 105.0052) (end 105.0902 105.6685) (width 0.2) (layer "B.Cu") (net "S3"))
 (segment (start 105.0902 106.5086) (end 106.7299 108.1483) (width 0.2) (layer "B.Cu") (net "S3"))
 (segment (start 107.3094 103.8459) (end 106.1501 105.0052) (width 0.2) (layer "B.Cu") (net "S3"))
 (segment (start 118.858 105.0552) (end 119.236 105.0552) (width 0.2) (layer "B.Cu") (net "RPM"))
 (segment (start 119.8414 107.3569) (end 119.05 108.1483) (width 0.2) (layer "B.Cu") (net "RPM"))
 (segment (start 119.8414 105.6606) (end 119.8414 107.3569) (width 0.2) (layer "B.Cu") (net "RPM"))
 (segment (start 119.05 109.625) (end 119.05 108.1483) (width 0.2) (layer "B.Cu") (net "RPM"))
 (segment (start 119.236 105.0552) (end 119.8414 105.6606) (width 0.2) (layer "B.Cu") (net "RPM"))
 (segment (start 117.55 102.29) (end 117.55 103.7472) (width 0.2) (layer "B.Cu") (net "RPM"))
 (segment (start 116.28 101.02) (end 117.55 102.29) (width 0.2) (layer "B.Cu") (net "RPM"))
 (segment (start 117.55 103.7472) (end 118.858 105.0552) (width 0.2) (layer "B.Cu") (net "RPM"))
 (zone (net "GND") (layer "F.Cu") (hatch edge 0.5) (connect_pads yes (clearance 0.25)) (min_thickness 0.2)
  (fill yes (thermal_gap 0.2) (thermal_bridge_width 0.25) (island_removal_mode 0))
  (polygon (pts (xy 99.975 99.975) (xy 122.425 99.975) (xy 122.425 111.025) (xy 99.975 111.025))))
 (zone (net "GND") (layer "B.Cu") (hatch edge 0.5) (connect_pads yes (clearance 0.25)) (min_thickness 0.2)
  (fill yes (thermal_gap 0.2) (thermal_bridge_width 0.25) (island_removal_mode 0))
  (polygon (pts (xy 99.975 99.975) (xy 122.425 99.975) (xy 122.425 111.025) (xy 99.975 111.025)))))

